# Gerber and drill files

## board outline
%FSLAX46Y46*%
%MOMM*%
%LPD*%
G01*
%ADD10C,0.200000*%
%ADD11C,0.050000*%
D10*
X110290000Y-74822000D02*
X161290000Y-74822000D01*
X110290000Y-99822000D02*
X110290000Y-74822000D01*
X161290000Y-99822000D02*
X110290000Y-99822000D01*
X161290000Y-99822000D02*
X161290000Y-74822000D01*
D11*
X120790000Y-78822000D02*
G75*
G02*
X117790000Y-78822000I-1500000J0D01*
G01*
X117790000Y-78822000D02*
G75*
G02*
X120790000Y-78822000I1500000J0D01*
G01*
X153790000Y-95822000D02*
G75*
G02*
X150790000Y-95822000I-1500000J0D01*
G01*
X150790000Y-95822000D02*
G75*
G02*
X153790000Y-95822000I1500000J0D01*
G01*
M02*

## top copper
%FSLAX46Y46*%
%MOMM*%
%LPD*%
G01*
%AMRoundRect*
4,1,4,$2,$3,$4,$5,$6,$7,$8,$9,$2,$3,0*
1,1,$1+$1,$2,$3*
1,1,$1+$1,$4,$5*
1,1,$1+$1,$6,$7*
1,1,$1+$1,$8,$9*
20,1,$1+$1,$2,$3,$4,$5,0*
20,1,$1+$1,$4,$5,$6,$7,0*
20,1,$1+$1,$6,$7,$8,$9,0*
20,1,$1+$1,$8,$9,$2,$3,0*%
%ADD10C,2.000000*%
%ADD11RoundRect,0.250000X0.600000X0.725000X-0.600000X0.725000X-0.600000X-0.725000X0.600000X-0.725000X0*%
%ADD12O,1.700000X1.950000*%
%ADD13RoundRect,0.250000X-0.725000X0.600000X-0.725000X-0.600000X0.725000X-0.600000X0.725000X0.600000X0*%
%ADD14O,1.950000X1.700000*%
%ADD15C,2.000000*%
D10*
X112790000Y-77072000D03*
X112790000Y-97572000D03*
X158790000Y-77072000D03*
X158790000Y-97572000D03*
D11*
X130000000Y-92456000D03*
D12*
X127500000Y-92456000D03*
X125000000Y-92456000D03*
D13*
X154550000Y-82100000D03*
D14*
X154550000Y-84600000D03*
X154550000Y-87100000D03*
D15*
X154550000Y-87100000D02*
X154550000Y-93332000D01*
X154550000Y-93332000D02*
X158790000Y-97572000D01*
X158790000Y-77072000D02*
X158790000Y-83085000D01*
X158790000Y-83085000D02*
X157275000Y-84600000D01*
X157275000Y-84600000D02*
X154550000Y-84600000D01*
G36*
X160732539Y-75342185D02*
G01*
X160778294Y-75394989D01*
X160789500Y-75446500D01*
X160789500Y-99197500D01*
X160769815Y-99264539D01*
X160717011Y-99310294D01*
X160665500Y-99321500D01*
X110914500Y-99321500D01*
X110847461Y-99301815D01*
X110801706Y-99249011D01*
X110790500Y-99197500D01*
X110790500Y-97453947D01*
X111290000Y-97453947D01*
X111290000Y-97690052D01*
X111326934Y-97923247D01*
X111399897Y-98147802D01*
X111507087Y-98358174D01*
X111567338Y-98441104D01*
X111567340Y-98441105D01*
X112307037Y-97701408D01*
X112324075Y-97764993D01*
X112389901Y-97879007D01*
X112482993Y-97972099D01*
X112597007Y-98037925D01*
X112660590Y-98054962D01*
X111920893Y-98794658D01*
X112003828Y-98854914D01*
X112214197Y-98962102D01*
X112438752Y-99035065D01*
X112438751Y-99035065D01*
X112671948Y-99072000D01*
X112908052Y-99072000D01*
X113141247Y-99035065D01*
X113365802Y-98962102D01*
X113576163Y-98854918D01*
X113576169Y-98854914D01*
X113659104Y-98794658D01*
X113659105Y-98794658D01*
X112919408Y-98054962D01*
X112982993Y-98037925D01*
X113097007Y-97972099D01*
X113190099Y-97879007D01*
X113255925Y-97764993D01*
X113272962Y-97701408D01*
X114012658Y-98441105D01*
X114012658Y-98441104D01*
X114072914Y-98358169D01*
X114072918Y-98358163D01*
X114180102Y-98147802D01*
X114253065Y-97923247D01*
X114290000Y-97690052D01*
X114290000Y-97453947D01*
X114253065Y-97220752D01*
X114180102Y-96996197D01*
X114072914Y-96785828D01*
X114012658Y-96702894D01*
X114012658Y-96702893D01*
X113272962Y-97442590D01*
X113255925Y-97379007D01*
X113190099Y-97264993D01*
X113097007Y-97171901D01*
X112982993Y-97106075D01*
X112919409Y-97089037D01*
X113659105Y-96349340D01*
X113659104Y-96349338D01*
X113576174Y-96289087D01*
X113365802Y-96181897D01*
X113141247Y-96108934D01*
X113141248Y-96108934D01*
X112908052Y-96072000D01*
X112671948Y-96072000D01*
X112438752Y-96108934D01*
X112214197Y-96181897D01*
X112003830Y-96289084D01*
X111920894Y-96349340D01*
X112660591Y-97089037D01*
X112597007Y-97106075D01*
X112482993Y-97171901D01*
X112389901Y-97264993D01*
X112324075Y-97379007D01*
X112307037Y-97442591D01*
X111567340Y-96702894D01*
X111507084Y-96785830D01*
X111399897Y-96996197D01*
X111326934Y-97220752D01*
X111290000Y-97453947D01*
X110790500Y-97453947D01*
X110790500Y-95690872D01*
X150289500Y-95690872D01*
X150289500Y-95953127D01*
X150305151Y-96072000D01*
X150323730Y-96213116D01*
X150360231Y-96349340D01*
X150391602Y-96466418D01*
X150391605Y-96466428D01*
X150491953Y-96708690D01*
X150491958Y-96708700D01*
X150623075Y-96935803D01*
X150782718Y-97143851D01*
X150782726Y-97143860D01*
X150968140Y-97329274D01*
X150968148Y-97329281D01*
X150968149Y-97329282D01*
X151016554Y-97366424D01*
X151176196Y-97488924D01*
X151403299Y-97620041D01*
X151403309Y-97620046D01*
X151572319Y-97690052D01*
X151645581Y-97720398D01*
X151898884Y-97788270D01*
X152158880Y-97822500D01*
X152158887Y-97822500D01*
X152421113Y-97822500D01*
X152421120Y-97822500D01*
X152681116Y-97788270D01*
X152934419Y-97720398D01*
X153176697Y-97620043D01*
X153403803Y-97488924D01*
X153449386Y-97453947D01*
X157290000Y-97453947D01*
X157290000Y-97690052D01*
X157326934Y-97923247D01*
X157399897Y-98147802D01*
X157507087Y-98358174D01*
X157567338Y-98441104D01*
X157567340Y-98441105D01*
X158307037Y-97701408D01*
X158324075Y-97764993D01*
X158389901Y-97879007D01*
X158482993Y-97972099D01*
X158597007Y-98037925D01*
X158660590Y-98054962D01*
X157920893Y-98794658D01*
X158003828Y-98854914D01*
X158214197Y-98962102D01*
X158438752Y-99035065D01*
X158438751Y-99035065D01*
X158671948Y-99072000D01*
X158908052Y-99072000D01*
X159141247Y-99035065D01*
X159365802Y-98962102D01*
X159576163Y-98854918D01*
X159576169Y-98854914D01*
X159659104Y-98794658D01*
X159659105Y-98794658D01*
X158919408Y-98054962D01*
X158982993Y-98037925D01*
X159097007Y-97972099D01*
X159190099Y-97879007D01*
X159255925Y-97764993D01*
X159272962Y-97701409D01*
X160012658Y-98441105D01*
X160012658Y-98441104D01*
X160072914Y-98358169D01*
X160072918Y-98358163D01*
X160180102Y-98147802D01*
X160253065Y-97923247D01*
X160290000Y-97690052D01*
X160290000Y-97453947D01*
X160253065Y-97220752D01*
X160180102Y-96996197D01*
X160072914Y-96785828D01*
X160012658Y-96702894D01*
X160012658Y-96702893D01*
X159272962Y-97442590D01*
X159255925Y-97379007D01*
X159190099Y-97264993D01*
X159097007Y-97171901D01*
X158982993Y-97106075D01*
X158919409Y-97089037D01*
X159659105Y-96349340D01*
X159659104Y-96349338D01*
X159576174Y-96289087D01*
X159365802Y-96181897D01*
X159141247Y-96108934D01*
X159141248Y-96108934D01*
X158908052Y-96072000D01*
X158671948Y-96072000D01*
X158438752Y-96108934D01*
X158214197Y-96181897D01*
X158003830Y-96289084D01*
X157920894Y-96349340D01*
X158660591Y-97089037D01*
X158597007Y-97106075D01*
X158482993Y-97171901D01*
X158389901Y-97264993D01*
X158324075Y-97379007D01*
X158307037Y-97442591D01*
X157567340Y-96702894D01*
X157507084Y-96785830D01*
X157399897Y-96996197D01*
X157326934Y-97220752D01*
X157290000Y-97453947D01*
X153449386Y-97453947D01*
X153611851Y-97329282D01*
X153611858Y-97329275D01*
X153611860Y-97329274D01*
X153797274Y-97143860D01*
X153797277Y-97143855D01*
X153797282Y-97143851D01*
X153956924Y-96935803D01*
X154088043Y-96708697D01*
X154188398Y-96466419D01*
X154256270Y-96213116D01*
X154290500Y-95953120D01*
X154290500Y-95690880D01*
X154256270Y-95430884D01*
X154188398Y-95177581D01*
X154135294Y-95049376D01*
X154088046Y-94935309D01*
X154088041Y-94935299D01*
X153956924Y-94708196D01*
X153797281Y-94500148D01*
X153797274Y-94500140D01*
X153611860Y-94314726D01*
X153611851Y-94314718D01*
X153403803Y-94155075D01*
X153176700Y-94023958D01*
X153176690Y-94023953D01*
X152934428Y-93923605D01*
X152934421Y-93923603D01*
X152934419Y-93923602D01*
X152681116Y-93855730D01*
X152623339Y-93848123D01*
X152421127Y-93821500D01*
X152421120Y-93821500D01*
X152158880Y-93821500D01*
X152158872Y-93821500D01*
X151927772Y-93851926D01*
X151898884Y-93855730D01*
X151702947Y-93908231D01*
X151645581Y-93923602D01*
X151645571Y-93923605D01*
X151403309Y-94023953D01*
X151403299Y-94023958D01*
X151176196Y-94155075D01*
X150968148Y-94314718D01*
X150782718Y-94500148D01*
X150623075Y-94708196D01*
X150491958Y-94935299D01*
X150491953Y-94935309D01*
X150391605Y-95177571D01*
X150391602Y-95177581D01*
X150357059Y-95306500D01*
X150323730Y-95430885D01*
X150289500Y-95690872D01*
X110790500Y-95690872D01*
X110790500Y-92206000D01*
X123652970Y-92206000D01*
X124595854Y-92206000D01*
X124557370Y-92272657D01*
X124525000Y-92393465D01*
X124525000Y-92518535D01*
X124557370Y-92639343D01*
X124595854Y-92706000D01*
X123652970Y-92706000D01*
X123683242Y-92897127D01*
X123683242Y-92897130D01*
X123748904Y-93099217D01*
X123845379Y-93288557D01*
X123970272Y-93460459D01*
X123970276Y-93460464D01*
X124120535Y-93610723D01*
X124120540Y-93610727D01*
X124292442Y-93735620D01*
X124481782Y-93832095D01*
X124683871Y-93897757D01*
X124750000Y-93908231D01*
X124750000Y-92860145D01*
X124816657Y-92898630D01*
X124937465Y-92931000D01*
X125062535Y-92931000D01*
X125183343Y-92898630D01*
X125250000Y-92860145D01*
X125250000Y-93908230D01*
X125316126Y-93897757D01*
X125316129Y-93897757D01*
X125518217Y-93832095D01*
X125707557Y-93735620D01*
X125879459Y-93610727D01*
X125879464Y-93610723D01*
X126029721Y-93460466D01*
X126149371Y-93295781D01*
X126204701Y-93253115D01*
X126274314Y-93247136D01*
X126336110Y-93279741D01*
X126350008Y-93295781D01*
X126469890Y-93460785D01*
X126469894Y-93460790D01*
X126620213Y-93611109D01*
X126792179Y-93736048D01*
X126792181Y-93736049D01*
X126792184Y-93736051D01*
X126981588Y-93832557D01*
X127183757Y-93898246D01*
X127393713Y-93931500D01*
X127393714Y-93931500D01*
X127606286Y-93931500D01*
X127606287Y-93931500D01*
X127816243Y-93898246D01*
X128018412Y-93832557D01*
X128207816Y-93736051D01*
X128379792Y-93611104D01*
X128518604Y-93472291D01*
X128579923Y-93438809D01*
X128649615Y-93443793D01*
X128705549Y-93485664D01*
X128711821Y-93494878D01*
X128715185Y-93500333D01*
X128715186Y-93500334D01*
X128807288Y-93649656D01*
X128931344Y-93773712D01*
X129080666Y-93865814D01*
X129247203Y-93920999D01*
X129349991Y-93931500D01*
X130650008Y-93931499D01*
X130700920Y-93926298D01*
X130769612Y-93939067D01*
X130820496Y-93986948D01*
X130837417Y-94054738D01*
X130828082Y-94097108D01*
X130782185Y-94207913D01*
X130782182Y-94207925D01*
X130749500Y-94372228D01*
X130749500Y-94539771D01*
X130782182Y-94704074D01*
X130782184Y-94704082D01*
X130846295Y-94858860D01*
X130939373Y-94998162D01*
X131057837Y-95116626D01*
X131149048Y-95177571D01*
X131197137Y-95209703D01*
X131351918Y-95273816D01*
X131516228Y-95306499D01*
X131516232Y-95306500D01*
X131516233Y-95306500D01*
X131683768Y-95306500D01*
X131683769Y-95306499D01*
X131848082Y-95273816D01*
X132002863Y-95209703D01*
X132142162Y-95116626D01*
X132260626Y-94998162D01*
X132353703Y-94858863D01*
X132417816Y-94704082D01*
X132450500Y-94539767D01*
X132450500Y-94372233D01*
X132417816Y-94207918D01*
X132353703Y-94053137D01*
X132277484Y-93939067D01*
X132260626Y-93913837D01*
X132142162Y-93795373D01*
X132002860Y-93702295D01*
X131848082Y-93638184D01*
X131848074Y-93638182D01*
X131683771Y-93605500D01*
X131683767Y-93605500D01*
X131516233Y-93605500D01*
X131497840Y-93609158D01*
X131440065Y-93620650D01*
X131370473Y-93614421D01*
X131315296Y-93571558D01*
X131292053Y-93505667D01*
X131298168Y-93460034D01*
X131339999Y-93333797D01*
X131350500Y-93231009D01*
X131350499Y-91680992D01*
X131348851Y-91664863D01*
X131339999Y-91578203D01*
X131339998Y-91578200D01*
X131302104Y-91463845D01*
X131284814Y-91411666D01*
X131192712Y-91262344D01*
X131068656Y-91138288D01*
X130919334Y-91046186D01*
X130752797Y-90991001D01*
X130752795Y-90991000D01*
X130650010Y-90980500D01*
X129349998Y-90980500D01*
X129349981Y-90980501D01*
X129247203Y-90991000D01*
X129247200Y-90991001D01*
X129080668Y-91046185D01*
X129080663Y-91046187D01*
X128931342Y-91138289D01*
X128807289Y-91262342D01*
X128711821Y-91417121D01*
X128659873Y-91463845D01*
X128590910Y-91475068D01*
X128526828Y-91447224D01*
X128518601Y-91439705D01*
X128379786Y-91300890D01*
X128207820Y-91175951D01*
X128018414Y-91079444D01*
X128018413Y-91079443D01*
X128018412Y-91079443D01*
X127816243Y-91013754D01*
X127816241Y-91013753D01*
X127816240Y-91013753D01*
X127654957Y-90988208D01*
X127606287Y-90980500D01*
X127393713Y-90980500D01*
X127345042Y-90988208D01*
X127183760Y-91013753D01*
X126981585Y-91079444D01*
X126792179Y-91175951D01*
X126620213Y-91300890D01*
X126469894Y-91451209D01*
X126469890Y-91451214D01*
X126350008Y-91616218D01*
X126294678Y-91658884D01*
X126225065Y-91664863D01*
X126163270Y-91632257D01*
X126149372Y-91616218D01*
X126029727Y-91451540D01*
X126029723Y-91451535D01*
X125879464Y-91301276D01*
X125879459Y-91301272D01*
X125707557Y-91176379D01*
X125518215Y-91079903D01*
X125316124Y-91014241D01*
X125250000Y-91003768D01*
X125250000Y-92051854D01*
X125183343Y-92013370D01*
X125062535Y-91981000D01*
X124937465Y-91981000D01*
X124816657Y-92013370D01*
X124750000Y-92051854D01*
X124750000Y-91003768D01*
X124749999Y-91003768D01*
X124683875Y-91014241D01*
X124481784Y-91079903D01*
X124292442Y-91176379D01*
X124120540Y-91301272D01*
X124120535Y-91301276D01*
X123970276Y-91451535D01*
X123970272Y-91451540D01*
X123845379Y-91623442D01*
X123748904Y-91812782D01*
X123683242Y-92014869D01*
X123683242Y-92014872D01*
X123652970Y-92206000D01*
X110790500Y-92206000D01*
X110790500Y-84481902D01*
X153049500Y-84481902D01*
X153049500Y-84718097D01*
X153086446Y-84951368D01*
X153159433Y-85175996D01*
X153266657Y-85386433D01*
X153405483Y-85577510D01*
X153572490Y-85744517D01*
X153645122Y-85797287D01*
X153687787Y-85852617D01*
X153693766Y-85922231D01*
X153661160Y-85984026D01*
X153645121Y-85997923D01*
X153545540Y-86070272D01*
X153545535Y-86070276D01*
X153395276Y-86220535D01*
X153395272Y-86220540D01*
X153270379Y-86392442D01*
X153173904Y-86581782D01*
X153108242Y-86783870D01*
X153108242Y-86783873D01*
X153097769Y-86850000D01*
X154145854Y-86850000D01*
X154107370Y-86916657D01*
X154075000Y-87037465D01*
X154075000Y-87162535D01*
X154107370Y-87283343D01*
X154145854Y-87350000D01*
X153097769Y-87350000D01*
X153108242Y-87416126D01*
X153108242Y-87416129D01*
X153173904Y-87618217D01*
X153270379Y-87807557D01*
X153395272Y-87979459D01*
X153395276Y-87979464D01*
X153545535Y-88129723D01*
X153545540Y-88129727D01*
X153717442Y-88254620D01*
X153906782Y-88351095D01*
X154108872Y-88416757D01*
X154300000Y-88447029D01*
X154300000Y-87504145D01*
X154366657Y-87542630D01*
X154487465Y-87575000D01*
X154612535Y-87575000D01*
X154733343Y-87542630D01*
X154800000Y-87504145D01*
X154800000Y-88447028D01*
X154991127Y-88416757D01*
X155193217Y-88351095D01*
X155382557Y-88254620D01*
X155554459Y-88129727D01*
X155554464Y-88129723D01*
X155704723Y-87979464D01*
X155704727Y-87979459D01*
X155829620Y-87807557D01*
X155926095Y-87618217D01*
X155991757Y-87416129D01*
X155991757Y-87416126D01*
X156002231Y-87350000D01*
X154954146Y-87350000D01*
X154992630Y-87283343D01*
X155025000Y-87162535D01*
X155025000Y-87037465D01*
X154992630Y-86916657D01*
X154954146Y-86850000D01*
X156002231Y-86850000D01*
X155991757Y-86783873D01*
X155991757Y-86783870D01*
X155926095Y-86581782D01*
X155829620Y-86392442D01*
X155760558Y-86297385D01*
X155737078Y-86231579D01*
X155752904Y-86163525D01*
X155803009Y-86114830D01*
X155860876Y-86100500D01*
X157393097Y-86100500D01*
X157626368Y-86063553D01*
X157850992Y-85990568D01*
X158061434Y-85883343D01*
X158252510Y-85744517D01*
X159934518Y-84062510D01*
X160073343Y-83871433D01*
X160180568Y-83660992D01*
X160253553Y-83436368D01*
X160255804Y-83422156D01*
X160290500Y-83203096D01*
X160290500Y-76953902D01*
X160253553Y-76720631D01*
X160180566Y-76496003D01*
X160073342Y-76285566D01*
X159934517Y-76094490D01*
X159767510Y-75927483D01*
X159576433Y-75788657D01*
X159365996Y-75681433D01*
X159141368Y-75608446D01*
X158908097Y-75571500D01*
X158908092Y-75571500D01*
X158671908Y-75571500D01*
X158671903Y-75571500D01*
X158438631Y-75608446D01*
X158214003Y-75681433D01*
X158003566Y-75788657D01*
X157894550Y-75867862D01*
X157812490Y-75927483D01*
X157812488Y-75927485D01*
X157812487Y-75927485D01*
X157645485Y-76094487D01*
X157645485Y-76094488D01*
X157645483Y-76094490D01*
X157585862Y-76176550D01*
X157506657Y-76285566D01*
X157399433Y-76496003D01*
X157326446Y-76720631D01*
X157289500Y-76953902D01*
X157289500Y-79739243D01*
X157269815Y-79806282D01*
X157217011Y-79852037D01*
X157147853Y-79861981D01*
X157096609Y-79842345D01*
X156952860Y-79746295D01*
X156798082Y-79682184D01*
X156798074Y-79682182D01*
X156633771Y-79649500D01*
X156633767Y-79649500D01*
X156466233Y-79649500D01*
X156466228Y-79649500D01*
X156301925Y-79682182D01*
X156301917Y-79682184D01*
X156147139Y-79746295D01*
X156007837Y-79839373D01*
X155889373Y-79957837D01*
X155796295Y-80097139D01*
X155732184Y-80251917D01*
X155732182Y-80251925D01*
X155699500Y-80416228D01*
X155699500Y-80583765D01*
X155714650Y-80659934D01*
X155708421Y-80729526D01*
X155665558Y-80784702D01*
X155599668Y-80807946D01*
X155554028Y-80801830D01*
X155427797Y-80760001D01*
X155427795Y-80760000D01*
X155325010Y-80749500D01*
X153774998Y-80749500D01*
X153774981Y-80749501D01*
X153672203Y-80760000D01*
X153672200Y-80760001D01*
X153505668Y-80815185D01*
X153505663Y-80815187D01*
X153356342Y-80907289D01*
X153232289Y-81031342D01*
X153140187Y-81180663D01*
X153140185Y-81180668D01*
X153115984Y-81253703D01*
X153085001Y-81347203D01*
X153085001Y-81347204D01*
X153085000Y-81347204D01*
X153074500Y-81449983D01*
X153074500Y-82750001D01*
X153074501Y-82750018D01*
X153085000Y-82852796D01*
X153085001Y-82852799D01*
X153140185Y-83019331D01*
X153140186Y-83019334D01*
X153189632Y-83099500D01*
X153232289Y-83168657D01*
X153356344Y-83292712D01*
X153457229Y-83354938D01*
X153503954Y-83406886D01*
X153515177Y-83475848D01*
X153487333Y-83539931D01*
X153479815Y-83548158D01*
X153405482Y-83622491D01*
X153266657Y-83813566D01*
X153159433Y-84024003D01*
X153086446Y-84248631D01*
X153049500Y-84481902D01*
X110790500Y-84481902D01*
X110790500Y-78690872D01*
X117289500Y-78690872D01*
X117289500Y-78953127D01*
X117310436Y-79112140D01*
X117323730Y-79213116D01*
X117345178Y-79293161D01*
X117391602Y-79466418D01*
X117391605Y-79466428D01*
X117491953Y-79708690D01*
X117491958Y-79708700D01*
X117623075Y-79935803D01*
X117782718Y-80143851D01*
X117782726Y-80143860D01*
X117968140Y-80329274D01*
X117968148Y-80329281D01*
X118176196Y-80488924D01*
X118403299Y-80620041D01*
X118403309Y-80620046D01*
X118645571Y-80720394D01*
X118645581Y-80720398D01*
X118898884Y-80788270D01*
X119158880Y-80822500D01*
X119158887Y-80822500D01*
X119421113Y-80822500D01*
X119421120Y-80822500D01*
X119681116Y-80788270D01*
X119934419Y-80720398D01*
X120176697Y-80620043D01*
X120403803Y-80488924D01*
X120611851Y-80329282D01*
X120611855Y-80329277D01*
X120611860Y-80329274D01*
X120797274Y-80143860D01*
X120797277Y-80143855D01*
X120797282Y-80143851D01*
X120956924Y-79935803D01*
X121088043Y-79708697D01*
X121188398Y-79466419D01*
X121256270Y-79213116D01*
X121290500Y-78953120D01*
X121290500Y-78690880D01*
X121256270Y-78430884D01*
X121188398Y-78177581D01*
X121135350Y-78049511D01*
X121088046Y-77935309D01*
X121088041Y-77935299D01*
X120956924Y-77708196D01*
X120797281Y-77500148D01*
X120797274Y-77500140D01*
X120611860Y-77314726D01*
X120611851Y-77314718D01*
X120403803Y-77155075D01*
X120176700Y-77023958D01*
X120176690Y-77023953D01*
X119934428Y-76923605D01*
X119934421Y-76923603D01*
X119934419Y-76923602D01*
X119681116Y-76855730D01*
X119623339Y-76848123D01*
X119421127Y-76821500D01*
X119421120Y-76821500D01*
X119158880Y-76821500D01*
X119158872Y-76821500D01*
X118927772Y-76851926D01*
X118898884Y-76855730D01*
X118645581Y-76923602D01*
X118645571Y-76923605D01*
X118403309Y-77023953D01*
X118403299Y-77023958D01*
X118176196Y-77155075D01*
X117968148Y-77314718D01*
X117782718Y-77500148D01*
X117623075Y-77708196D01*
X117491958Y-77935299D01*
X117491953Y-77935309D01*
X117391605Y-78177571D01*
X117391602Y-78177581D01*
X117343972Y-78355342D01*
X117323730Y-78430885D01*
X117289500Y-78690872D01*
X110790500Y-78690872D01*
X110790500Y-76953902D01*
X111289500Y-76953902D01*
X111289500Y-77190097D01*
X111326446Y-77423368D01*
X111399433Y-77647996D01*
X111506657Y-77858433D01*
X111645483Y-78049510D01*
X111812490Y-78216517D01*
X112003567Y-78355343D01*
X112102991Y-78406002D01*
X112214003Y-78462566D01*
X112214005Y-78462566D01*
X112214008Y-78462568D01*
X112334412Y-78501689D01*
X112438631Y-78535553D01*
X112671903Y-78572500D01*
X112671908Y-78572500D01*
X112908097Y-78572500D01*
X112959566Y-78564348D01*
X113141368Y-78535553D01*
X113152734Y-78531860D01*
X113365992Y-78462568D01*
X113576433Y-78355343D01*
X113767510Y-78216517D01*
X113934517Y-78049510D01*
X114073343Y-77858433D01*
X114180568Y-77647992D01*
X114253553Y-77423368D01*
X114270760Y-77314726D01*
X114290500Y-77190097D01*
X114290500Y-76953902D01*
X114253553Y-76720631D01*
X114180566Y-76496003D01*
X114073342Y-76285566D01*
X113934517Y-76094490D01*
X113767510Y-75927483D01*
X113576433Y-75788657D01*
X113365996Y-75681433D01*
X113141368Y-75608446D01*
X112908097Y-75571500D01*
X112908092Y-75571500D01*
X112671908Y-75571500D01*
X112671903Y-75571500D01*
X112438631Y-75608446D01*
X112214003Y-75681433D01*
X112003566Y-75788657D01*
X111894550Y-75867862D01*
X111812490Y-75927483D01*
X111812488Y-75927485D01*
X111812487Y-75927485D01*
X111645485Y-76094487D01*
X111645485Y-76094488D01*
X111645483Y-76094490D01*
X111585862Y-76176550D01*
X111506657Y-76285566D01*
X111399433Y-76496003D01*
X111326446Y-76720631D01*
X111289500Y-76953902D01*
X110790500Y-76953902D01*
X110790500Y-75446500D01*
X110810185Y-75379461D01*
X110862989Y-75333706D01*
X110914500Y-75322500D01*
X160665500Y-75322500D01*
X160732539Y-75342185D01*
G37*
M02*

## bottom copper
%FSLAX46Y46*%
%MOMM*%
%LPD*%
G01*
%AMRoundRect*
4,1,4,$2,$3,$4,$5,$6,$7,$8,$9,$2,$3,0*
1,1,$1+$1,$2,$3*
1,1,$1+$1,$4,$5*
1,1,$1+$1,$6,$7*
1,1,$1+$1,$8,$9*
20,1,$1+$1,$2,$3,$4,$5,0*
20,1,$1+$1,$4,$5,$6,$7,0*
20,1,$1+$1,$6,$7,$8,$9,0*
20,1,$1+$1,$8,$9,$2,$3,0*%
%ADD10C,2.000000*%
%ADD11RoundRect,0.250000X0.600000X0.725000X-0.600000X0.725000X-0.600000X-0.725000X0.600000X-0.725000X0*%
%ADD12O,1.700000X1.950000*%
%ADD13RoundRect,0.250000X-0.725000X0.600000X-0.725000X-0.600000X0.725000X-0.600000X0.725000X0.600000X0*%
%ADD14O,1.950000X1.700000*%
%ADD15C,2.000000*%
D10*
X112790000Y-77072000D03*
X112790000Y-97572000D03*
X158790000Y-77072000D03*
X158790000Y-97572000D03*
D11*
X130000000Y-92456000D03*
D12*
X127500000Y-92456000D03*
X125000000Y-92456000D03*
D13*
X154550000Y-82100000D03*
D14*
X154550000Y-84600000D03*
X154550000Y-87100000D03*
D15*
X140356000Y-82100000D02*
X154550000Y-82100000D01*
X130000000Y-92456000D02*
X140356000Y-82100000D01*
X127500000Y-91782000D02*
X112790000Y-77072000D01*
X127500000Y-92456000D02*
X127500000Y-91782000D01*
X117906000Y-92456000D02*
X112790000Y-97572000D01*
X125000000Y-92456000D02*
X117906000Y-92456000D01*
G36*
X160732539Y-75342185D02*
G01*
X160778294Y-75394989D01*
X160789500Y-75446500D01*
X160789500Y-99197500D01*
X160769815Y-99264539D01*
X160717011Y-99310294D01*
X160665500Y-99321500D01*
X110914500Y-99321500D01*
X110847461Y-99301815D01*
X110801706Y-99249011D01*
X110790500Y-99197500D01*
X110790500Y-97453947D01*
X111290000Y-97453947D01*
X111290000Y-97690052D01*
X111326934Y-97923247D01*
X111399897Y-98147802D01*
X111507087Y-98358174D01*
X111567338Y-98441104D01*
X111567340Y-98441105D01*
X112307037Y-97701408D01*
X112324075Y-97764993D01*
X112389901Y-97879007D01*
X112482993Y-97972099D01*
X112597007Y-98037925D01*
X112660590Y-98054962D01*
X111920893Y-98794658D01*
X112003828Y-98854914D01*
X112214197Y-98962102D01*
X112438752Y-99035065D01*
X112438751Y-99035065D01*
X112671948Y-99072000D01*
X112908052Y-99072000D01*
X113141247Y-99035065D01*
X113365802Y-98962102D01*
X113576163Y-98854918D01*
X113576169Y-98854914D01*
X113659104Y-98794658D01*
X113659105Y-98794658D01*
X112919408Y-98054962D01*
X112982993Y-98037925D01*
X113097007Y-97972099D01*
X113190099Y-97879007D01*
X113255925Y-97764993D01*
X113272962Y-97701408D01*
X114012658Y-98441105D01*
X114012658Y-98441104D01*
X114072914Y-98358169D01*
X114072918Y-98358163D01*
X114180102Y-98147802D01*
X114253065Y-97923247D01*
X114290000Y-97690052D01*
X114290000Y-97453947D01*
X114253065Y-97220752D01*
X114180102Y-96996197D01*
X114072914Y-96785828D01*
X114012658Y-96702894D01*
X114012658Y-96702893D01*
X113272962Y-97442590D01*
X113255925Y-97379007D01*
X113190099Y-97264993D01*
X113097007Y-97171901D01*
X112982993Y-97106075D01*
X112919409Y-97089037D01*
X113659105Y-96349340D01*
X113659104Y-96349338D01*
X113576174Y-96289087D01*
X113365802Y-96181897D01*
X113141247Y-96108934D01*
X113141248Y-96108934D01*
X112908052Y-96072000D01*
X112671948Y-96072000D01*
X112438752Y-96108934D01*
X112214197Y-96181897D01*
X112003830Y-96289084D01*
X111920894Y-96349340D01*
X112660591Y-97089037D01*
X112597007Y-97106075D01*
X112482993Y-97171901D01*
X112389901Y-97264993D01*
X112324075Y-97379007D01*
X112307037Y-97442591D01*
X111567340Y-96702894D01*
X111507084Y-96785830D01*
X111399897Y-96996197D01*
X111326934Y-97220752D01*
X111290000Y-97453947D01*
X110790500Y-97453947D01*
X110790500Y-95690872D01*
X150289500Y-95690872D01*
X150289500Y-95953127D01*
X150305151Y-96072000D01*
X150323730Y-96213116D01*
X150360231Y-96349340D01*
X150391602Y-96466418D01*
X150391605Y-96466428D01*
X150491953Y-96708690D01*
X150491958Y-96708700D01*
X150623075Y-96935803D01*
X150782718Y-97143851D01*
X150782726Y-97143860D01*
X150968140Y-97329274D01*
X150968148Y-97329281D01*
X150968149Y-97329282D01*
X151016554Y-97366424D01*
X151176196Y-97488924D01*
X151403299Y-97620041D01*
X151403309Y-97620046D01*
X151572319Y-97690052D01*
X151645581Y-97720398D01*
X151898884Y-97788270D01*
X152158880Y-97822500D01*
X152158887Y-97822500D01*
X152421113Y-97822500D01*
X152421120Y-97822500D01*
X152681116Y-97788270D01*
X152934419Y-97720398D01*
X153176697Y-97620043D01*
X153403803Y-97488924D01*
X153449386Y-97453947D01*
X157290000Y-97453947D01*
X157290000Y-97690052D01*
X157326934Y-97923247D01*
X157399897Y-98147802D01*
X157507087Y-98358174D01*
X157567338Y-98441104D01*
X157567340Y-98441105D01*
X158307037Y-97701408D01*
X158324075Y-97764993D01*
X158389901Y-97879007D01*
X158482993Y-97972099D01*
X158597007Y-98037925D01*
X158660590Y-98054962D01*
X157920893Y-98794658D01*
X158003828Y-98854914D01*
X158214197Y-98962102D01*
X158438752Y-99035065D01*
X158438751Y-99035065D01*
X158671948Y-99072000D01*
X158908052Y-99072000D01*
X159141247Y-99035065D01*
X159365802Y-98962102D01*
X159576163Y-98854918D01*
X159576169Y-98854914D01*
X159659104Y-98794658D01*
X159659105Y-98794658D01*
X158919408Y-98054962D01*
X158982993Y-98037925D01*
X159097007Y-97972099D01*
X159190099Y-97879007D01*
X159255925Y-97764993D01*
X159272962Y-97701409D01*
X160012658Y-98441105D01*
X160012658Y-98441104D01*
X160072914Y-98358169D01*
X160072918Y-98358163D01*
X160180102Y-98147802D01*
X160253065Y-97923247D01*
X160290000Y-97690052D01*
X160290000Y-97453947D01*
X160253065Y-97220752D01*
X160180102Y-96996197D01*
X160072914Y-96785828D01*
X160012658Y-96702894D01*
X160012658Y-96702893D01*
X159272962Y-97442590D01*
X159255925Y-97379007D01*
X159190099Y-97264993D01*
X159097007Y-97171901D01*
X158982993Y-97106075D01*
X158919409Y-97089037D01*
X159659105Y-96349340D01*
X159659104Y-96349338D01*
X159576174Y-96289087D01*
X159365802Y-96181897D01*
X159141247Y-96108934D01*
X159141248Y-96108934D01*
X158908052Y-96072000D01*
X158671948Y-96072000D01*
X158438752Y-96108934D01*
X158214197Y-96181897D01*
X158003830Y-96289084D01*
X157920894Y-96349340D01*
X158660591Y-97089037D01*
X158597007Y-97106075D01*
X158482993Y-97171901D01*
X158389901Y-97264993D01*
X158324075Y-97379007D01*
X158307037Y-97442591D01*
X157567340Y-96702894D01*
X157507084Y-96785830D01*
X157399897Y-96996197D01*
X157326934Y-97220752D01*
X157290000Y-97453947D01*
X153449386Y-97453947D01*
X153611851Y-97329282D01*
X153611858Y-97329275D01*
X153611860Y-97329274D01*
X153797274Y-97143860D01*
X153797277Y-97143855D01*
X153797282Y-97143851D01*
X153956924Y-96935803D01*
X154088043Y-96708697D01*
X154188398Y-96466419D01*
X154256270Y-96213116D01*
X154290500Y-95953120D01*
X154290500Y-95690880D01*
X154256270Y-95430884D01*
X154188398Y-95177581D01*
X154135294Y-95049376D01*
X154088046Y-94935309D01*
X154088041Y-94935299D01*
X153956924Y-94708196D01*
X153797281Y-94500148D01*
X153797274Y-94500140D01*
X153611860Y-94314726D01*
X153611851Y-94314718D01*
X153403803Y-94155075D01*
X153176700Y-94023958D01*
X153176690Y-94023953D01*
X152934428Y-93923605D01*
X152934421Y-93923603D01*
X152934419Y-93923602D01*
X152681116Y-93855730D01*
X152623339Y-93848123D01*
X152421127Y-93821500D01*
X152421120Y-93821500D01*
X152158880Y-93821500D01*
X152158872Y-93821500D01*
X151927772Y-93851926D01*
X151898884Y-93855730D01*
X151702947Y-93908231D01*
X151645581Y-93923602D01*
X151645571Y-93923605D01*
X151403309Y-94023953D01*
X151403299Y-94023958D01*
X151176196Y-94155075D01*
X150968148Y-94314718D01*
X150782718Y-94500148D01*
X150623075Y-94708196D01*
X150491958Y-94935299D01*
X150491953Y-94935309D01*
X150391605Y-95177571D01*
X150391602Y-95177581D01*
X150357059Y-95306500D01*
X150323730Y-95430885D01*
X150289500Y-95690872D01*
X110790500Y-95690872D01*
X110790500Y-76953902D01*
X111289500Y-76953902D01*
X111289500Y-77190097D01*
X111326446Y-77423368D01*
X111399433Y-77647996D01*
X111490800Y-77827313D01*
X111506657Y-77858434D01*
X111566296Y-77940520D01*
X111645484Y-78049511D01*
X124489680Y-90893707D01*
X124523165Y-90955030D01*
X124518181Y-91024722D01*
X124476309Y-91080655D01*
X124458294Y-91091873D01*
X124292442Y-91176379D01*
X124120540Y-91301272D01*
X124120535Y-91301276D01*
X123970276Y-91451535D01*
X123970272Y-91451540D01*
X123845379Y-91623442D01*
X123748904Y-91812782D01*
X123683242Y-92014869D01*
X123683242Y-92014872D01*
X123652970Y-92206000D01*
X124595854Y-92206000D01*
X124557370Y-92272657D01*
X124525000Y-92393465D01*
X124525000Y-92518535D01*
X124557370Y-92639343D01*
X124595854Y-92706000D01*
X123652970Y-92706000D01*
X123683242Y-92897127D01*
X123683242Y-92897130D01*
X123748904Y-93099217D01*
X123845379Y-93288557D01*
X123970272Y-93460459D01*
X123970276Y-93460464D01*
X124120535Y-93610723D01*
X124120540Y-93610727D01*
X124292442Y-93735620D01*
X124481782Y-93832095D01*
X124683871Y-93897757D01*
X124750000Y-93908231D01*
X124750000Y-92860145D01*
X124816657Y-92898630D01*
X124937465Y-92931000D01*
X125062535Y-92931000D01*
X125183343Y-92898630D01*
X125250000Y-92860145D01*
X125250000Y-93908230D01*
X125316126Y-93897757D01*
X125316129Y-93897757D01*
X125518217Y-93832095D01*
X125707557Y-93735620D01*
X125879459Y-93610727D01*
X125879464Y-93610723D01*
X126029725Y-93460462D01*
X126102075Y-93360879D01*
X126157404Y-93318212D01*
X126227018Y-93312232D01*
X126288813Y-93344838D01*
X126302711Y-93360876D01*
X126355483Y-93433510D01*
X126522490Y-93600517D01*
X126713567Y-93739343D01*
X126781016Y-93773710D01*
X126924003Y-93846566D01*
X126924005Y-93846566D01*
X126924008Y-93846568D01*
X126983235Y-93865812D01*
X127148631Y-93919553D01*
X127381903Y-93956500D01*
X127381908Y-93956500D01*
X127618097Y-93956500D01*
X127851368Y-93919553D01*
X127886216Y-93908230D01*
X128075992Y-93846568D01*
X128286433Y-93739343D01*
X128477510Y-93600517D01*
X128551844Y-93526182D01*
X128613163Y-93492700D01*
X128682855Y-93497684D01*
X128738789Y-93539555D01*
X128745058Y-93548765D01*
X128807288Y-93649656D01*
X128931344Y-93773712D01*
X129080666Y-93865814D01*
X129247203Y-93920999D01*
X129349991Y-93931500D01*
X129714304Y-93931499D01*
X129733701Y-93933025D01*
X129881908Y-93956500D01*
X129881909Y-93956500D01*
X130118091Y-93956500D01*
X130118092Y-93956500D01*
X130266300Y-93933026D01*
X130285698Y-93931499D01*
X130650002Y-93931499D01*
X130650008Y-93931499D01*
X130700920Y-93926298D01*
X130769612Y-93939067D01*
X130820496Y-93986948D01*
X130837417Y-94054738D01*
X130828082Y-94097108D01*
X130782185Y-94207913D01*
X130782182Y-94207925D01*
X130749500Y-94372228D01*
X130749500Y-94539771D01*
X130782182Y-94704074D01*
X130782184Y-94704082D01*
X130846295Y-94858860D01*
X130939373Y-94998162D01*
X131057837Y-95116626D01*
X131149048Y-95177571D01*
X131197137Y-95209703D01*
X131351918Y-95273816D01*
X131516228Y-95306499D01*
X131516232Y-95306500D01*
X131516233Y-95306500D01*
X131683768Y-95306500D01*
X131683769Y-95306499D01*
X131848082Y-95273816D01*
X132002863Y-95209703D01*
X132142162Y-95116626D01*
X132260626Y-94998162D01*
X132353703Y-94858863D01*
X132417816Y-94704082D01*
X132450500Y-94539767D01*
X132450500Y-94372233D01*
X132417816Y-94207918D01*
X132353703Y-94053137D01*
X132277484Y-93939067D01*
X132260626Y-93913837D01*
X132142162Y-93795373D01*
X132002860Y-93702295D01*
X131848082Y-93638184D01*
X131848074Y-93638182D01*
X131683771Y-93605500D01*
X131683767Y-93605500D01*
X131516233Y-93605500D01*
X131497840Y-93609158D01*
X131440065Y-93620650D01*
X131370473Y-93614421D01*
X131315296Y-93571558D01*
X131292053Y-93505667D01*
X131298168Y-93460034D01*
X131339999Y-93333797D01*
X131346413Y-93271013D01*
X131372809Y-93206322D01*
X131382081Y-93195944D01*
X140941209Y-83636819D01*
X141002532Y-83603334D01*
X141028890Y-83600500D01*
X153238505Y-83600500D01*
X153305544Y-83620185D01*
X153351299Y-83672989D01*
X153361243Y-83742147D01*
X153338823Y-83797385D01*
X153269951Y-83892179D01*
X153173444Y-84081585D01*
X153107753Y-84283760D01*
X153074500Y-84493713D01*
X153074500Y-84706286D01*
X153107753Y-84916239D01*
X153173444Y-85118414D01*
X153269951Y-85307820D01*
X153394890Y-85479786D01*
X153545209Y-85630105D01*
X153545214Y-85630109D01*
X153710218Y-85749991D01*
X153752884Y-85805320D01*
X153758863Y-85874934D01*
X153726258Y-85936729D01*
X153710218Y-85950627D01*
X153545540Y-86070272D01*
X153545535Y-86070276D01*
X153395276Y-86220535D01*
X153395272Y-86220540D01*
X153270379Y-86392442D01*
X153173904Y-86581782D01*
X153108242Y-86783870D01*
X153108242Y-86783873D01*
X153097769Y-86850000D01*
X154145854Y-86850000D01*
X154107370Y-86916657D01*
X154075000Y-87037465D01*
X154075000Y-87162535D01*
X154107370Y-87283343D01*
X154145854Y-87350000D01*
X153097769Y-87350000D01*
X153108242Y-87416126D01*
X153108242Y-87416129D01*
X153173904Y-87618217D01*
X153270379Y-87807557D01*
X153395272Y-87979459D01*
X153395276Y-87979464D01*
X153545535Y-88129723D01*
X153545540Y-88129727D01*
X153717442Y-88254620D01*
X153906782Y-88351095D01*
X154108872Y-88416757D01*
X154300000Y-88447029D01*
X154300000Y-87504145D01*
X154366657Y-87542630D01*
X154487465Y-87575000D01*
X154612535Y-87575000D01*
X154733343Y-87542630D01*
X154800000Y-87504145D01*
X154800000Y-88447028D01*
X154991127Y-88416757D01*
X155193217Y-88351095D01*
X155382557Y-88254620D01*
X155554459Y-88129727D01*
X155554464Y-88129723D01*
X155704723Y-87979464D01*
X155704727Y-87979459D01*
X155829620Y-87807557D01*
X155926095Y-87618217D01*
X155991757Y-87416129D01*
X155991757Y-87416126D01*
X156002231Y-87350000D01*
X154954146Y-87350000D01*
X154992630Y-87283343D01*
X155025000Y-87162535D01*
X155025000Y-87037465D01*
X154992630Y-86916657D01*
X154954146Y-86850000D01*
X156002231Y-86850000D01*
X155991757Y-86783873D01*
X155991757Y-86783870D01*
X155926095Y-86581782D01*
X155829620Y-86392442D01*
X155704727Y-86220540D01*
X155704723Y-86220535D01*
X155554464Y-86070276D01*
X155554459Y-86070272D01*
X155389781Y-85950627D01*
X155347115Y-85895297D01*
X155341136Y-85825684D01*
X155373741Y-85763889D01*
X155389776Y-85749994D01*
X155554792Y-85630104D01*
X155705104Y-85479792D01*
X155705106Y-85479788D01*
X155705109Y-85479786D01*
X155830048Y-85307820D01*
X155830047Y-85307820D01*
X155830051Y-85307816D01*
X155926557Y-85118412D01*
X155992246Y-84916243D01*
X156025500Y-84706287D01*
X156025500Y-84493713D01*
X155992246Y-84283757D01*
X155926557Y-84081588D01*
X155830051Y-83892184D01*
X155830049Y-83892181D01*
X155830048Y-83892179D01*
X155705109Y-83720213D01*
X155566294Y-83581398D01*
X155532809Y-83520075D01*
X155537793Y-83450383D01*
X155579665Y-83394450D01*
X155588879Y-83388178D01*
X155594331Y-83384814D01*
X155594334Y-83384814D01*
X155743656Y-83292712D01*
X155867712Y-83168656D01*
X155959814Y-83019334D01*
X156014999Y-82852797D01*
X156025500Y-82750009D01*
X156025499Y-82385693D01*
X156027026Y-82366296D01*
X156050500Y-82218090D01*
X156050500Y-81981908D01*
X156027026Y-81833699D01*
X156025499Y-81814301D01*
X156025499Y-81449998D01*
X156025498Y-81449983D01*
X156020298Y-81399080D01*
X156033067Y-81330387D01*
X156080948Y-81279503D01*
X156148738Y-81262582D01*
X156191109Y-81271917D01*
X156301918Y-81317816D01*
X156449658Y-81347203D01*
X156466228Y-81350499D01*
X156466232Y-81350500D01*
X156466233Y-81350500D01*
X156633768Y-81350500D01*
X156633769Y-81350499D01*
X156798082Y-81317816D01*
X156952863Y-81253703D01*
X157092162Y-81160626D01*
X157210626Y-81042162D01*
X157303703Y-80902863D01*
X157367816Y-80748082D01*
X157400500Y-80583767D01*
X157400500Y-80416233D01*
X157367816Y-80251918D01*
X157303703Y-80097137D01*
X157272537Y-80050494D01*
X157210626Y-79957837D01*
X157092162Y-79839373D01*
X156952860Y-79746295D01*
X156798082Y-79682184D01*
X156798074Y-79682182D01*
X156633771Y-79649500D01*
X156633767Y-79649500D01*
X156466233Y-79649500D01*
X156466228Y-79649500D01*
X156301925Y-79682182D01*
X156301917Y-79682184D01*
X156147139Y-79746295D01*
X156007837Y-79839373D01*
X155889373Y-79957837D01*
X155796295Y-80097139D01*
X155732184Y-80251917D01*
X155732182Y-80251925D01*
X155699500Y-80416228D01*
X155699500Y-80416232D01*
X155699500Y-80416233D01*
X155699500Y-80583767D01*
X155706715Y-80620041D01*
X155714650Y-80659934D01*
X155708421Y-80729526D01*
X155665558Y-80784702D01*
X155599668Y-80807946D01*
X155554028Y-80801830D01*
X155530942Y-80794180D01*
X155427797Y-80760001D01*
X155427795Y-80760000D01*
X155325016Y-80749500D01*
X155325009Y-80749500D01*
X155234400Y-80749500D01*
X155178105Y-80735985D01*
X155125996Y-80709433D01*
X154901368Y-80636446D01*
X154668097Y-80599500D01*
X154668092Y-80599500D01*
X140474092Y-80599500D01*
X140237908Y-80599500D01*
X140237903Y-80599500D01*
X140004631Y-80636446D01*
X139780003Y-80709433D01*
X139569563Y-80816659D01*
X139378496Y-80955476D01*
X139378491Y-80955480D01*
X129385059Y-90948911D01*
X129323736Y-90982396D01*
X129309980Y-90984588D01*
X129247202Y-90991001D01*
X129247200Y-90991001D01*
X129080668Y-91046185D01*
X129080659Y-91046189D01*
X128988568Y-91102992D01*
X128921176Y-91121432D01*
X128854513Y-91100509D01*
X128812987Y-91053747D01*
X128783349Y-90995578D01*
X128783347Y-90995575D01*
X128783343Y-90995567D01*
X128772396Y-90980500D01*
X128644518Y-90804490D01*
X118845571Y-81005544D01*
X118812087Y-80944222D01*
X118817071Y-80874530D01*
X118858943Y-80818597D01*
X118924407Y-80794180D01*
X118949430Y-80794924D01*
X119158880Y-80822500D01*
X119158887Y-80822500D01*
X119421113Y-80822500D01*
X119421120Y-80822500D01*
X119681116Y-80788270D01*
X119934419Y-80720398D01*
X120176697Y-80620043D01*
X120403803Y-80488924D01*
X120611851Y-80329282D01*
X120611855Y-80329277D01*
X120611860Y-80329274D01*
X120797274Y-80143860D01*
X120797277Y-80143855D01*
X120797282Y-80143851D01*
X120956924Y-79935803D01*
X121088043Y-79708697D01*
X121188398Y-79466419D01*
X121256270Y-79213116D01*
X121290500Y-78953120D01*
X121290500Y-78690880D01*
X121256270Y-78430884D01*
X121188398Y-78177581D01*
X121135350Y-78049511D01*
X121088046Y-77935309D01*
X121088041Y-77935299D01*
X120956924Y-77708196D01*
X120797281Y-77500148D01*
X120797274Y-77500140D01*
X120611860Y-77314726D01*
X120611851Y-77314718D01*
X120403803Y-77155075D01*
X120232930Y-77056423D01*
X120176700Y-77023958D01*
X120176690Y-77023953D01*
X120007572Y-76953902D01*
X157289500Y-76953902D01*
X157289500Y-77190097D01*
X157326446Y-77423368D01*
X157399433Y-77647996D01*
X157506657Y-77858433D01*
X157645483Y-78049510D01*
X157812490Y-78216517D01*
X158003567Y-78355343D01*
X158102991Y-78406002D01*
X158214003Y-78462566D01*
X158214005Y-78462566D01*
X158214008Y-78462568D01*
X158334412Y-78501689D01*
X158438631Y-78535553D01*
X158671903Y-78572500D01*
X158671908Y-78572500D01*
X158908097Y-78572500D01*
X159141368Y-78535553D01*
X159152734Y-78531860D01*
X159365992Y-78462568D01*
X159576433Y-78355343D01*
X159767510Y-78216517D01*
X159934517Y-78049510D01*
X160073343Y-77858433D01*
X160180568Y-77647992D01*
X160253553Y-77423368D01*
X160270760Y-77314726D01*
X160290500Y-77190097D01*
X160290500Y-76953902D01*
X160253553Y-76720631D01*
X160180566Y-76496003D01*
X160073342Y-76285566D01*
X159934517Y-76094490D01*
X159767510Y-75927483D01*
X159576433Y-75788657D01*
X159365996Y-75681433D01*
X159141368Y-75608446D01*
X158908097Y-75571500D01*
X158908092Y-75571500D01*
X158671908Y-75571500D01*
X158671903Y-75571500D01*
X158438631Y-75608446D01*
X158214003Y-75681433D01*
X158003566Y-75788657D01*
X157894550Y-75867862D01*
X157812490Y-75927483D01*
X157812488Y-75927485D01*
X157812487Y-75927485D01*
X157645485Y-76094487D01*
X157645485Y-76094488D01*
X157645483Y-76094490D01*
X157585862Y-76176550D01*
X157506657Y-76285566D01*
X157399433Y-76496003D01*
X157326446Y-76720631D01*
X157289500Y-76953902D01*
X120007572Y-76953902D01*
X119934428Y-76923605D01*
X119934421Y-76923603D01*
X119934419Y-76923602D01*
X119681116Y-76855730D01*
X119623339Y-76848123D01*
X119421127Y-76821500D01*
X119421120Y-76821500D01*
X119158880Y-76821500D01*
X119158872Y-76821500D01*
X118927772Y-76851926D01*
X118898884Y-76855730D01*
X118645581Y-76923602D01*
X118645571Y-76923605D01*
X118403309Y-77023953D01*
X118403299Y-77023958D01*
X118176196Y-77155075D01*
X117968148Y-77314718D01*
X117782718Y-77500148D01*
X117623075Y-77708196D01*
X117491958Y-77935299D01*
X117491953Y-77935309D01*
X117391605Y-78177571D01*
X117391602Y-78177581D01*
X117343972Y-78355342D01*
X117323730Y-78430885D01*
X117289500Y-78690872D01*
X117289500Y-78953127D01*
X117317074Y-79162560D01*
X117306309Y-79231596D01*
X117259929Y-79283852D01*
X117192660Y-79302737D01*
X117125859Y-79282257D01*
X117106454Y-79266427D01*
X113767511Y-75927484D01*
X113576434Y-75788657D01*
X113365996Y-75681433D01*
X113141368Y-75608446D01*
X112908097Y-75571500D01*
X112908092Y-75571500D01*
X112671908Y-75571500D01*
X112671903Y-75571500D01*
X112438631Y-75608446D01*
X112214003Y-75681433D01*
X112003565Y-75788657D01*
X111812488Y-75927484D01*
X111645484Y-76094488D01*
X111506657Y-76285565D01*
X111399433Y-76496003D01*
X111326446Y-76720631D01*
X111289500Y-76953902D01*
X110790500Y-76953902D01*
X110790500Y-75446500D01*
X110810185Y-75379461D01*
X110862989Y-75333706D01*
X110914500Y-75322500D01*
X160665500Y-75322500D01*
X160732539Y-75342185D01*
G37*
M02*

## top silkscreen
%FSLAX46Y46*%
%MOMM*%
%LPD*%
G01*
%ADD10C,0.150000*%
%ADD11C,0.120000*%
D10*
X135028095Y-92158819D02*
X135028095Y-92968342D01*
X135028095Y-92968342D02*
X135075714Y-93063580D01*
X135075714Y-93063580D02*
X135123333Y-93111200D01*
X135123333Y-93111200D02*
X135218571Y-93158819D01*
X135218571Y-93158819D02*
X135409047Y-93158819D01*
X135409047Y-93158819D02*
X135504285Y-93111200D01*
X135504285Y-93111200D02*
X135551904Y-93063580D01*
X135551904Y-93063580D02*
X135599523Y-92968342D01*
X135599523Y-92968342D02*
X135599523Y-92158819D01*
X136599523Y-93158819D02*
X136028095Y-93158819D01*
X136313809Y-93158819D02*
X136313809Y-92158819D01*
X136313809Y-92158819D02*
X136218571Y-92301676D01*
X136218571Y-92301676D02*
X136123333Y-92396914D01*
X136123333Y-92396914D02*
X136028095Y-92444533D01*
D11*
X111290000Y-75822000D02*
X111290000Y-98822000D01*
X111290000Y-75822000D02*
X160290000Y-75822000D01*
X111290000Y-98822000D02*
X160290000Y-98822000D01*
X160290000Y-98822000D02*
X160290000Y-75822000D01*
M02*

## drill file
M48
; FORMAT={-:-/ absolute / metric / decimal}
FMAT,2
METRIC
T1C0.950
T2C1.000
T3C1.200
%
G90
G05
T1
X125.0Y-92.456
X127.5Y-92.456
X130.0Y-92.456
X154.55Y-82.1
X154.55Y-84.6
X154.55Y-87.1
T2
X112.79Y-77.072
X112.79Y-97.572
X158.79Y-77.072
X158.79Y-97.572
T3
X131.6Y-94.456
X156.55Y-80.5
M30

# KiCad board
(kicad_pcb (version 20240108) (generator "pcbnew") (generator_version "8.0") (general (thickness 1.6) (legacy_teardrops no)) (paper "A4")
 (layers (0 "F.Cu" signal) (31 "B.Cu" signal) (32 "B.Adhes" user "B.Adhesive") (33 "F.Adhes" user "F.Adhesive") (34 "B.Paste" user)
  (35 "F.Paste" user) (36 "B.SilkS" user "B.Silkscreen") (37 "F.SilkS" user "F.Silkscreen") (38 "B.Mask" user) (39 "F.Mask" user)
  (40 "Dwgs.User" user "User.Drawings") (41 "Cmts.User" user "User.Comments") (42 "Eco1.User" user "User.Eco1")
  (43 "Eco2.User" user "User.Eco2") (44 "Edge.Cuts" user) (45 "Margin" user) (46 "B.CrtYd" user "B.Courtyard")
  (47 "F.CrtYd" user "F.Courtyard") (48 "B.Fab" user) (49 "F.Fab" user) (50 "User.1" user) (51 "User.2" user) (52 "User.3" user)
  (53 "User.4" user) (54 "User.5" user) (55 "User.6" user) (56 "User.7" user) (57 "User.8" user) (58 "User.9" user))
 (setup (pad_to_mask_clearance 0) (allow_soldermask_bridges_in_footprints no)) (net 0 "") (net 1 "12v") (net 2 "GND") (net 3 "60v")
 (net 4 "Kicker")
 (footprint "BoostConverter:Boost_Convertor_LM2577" (layer "F.Cu") (at 135.79 87.322)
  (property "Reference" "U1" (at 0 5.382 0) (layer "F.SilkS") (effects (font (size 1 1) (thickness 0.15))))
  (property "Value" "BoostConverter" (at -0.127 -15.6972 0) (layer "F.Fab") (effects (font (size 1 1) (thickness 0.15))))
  (fp_line (start -24.5 -11.5) (end -24.5 11.5) (stroke (width 0.12) (type solid)) (layer "F.SilkS"))
  (fp_line (start -24.5 -11.5) (end 24.5 -11.5) (stroke (width 0.12) (type solid)) (layer "F.SilkS"))
  (fp_line (start -24.5 11.5) (end 24.5 11.5) (stroke (width 0.12) (type solid)) (layer "F.SilkS"))
  (fp_line (start 24.5 11.5) (end 24.5 -11.5) (stroke (width 0.12) (type solid)) (layer "F.SilkS"))
  (fp_circle (center -16.5 -8.5) (end -15 -8.5) (stroke (width 0.05) (type default)) (fill none) (layer "Edge.Cuts"))
  (fp_circle (center 16.5 8.5) (end 18 8.5) (stroke (width 0.05) (type default)) (fill none) (layer "Edge.Cuts"))
  (pad "1" thru_hole circle (at -23 -10.25) (size 2 2) (drill 1) (layers "*.Cu" "*.Mask") (remove_unused_layers no) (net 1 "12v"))
  (pad "2" thru_hole circle (at -23 10.25) (size 2 2) (drill 1) (layers "*.Cu" "*.Mask") (remove_unused_layers no) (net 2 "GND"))
  (pad "3" thru_hole circle (at 23 -10.25) (size 2 2) (drill 1) (layers "*.Cu" "*.Mask") (remove_unused_layers no) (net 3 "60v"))
  (pad "4" thru_hole circle (at 23 10.25) (size 2 2) (drill 1) (layers "*.Cu" "*.Mask") (remove_unused_layers no) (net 2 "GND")))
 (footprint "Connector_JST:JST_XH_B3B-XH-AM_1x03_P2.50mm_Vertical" (layer "B.Cu") (at 130 92.456 180)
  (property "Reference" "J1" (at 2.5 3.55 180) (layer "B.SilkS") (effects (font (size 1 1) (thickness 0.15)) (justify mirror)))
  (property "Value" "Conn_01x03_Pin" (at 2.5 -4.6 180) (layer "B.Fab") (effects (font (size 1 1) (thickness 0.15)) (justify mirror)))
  (pad "" np_thru_hole circle (at -1.6 -2 180) (size 1.2 1.2) (drill 1.2) (layers "*.Cu" "*.Mask"))
  (pad "1" thru_hole roundrect (at 0 0 180) (size 1.7 1.95) (drill 0.95) (layers "*.Cu" "*.Mask") (remove_unused_layers no)
   (roundrect_rratio 0.147059) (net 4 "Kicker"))
  (pad "2" thru_hole oval (at 2.5 0 180) (size 1.7 1.95) (drill 0.95) (layers "*.Cu" "*.Mask") (remove_unused_layers no) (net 1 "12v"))
  (pad "3" thru_hole oval (at 5 0 180) (size 1.7 1.95) (drill 0.95) (layers "*.Cu" "*.Mask") (remove_unused_layers no) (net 2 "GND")))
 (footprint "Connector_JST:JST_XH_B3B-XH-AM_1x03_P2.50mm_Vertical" (layer "B.Cu") (at 154.55 82.1 -90)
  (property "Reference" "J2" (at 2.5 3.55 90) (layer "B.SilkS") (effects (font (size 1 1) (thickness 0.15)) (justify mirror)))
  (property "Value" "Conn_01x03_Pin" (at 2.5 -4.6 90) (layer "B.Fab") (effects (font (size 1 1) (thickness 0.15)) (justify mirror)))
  (pad "" np_thru_hole circle (at -1.6 -2 270) (size 1.2 1.2) (drill 1.2) (layers "*.Cu" "*.Mask"))
  (pad "1" thru_hole roundrect (at 0 0 270) (size 1.7 1.95) (drill 0.95) (layers "*.Cu" "*.Mask") (remove_unused_layers no)
   (roundrect_rratio 0.147059) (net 4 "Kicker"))
  (pad "2" thru_hole oval (at 2.5 0 270) (size 1.7 1.95) (drill 0.95) (layers "*.Cu" "*.Mask") (remove_unused_layers no) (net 3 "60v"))
  (pad "3" thru_hole oval (at 5 0 270) (size 1.7 1.95) (drill 0.95) (layers "*.Cu" "*.Mask") (remove_unused_layers no) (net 2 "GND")))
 (gr_line (start 110.29 74.822) (end 161.29 74.822) (stroke (width 0.2) (type solid)) (layer "Edge.Cuts"))
 (gr_line (start 110.29 99.822) (end 110.29 74.822) (stroke (width 0.2) (type solid)) (layer "Edge.Cuts"))
 (gr_line (start 161.29 99.822) (end 110.29 99.822) (stroke (width 0.2) (type solid)) (layer "Edge.Cuts"))
 (gr_line (start 161.29 99.822) (end 161.29 74.822) (stroke (width 0.2) (type solid)) (layer "Edge.Cuts"))
 (segment (start 140.356 82.1) (end 154.55 82.1) (width 2) (layer "B.Cu") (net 4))
 (segment (start 130 92.456) (end 140.356 82.1) (width 2) (layer "B.Cu") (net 4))
 (segment (start 127.5 91.782) (end 112.79 77.072) (width 2) (layer "B.Cu") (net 1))
 (segment (start 127.5 92.456) (end 127.5 91.782) (width 2) (layer "B.Cu") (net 1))
 (segment (start 154.55 87.1) (end 154.55 93.332) (width 2) (layer "F.Cu") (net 2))
 (segment (start 154.55 93.332) (end 158.79 97.572) (width 2) (layer "F.Cu") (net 2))
 (segment (start 117.906 92.456) (end 112.79 97.572) (width 2) (layer "B.Cu") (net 2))
 (segment (start 125 92.456) (end 117.906 92.456) (width 2) (layer "B.Cu") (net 2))
 (segment (start 158.79 77.072) (end 158.79 83.085) (width 2) (layer "F.Cu") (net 3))
 (segment (start 158.79 83.085) (end 157.275 84.6) (width 2) (layer "F.Cu") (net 3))
 (segment (start 157.275 84.6) (end 154.55 84.6) (width 2) (layer "F.Cu") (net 3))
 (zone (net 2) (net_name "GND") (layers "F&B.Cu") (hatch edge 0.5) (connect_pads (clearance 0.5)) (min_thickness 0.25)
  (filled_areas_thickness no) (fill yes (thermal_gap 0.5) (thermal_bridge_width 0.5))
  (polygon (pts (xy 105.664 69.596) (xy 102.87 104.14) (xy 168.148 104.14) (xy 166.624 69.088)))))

